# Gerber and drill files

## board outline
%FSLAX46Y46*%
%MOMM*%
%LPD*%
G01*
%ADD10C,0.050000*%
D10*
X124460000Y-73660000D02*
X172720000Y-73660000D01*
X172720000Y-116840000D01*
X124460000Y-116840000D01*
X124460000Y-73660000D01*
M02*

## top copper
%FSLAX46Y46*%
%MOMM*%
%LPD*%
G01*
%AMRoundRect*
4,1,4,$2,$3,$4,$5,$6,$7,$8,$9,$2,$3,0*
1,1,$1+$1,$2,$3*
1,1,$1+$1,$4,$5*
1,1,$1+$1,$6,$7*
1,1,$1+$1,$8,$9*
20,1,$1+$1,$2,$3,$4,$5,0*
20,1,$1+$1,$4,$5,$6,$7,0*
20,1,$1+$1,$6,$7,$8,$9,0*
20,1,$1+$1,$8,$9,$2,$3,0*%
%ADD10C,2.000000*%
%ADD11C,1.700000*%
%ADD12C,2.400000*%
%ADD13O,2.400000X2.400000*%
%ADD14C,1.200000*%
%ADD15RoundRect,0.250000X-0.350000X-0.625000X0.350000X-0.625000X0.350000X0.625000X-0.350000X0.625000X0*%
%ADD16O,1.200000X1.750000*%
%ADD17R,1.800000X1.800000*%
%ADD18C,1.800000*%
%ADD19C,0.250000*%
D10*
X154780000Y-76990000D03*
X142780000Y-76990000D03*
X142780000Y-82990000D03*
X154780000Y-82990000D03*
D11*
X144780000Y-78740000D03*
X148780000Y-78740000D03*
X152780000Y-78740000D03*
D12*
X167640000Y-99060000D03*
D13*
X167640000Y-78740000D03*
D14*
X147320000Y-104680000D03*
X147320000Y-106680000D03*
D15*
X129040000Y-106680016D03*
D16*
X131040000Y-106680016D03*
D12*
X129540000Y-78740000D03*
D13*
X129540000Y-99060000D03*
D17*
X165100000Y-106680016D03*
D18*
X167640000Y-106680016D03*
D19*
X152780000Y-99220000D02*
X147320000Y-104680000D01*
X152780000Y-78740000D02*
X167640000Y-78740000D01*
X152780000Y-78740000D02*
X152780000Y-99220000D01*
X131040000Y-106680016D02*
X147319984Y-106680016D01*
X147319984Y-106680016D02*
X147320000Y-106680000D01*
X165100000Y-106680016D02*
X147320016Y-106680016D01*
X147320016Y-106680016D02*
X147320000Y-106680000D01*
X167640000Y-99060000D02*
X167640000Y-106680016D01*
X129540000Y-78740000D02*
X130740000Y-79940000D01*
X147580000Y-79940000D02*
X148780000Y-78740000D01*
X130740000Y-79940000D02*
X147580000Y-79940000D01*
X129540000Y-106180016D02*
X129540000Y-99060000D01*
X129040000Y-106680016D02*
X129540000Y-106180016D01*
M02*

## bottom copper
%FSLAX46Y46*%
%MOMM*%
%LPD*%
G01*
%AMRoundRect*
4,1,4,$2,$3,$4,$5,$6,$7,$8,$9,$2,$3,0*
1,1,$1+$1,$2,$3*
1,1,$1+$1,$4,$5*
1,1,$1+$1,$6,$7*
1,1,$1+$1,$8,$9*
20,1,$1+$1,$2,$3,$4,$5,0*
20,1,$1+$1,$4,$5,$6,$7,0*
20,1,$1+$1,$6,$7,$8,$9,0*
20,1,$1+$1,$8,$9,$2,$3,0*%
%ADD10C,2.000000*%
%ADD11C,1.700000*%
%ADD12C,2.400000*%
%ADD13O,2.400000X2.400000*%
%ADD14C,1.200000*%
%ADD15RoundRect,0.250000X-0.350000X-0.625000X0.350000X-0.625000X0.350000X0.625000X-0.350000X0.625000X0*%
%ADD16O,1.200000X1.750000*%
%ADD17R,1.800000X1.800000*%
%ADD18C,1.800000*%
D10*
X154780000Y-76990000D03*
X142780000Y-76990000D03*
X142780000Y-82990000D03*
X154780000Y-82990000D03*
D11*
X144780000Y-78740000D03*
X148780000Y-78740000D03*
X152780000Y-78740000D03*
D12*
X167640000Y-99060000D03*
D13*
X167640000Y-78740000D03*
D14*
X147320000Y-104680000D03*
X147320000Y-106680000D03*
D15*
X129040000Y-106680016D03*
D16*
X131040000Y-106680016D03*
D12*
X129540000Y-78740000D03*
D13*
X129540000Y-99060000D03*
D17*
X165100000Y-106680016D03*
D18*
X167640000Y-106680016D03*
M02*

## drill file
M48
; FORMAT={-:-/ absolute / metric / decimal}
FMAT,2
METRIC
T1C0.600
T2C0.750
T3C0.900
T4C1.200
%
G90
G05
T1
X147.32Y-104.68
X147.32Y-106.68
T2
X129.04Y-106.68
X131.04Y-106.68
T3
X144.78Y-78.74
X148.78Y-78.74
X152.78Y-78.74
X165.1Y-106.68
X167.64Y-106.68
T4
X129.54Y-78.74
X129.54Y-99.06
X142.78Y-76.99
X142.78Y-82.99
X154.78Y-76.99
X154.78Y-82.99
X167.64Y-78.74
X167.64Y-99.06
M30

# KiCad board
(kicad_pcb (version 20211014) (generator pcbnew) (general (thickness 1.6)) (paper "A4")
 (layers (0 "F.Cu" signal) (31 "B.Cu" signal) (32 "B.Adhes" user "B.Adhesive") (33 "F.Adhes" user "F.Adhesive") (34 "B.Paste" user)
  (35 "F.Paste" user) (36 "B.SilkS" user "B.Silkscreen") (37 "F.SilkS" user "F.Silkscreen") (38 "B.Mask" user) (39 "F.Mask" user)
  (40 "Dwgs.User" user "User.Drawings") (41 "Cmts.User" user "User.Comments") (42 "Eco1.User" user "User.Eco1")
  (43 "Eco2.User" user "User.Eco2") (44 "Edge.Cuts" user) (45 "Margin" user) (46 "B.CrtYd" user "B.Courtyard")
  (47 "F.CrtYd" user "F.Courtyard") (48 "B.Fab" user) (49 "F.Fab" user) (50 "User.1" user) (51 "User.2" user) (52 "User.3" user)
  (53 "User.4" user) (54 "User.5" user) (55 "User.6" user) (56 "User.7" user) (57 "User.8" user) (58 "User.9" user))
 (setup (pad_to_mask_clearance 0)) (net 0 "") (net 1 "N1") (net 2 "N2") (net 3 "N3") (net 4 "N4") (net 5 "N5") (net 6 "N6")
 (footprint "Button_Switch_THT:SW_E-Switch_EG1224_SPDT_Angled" (layer "F.Cu") (at 144.78 78.74)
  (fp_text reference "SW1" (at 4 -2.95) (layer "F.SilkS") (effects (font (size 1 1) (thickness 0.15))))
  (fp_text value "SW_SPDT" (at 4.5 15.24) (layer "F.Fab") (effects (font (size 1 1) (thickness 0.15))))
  (pad "" thru_hole circle (at 10 -1.75) (size 2 2) (drill 1.2) (layers *.Cu *.Mask))
  (pad "" thru_hole circle (at -2 -1.75) (size 2 2) (drill 1.2) (layers *.Cu *.Mask))
  (pad "" thru_hole circle (at -2 4.25) (size 2 2) (drill 1.2) (layers *.Cu *.Mask))
  (pad "" thru_hole circle (at 10 4.25) (size 2 2) (drill 1.2) (layers *.Cu *.Mask))
  (pad "1" thru_hole circle (at 0 0) (size 1.7 1.7) (drill 0.9) (layers *.Cu *.Mask) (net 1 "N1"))
  (pad "2" thru_hole circle (at 4 0) (size 1.7 1.7) (drill 0.9) (layers *.Cu *.Mask) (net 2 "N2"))
  (pad "3" thru_hole circle (at 8 0) (size 1.7 1.7) (drill 0.9) (layers *.Cu *.Mask) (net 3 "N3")))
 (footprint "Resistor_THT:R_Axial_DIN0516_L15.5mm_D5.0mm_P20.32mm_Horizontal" (layer "F.Cu") (at 167.64 99.06 90)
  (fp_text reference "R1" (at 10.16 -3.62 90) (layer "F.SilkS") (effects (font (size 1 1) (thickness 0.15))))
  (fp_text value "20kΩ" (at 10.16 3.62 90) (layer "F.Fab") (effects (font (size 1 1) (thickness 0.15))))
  (pad "1" thru_hole circle (at 0 0 90) (size 2.4 2.4) (drill 1.2) (layers *.Cu *.Mask) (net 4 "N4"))
  (pad "2" thru_hole oval (at 20.32 0 90) (size 2.4 2.4) (drill 1.2) (layers *.Cu *.Mask) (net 3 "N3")))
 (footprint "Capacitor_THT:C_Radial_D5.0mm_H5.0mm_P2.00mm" (layer "F.Cu") (at 147.32 104.68 -90)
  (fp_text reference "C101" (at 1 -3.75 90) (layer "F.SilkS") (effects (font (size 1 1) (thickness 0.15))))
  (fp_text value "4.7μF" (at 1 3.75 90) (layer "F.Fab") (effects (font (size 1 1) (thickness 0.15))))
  (pad "1" thru_hole circle (at 0 0 270) (size 1.2 1.2) (drill 0.6) (layers *.Cu *.Mask) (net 3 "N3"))
  (pad "2" thru_hole circle (at 2 0 270) (size 1.2 1.2) (drill 0.6) (layers *.Cu *.Mask) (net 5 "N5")))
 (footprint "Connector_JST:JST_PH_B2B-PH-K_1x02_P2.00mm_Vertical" (layer "F.Cu") (at 129.04 106.680016)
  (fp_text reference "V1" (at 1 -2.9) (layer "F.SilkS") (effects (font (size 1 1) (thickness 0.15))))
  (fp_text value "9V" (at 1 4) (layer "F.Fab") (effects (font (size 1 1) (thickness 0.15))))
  (pad "1" thru_hole roundrect (at 0 0) (size 1.2 1.75) (drill 0.75) (layers *.Cu *.Mask) (roundrect_rratio 0.208333) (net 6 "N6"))
  (pad "2" thru_hole oval (at 2 0) (size 1.2 1.75) (drill 0.75) (layers *.Cu *.Mask) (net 5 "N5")))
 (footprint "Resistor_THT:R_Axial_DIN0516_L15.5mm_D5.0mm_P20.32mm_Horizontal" (layer "F.Cu") (at 129.54 78.74 -90)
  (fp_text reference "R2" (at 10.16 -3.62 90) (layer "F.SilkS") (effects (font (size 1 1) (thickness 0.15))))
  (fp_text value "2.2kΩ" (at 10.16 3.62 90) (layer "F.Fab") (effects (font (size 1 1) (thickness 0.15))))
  (pad "1" thru_hole circle (at 0 0 270) (size 2.4 2.4) (drill 1.2) (layers *.Cu *.Mask) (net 2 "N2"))
  (pad "2" thru_hole oval (at 20.32 0 270) (size 2.4 2.4) (drill 1.2) (layers *.Cu *.Mask) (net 6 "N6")))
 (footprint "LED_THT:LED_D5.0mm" (layer "F.Cu") (at 165.1 106.680016)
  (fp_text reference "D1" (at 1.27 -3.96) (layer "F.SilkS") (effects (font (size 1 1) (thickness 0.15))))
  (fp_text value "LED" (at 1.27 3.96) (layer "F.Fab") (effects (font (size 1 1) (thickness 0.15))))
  (pad "1" thru_hole rect (at 0 0) (size 1.8 1.8) (drill 0.9) (layers *.Cu *.Mask) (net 5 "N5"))
  (pad "2" thru_hole circle (at 2.54 0) (size 1.8 1.8) (drill 0.9) (layers *.Cu *.Mask) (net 4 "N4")))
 (gr_rect (start 124.46 73.66) (end 172.72 116.84) (layer "Edge.Cuts") (width 0.05) (fill none))
 (segment (start 152.78 99.22) (end 147.32 104.68) (width 0.25) (layer "F.Cu") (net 3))
 (segment (start 152.78 78.74) (end 167.64 78.74) (width 0.25) (layer "F.Cu") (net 3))
 (segment (start 152.78 78.74) (end 152.78 99.22) (width 0.25) (layer "F.Cu") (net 3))
 (segment (start 131.04 106.680016) (end 147.319984 106.680016) (width 0.25) (layer "F.Cu") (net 5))
 (segment (start 147.319984 106.680016) (end 147.32 106.68) (width 0.25) (layer "F.Cu") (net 5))
 (segment (start 165.1 106.680016) (end 147.320016 106.680016) (width 0.25) (layer "F.Cu") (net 5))
 (segment (start 147.320016 106.680016) (end 147.32 106.68) (width 0.25) (layer "F.Cu") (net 5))
 (segment (start 167.64 99.06) (end 167.64 106.680016) (width 0.25) (layer "F.Cu") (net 4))
 (segment (start 129.54 78.74) (end 130.74 79.94) (width 0.25) (layer "F.Cu") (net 2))
 (segment (start 147.58 79.94) (end 148.78 78.74) (width 0.25) (layer "F.Cu") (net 2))
 (segment (start 130.74 79.94) (end 147.58 79.94) (width 0.25) (layer "F.Cu") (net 2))
 (segment (start 129.54 106.180016) (end 129.54 99.06) (width 0.25) (layer "F.Cu") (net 6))
 (segment (start 129.04 106.680016) (end 129.54 106.180016) (width 0.25) (layer "F.Cu") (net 6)))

